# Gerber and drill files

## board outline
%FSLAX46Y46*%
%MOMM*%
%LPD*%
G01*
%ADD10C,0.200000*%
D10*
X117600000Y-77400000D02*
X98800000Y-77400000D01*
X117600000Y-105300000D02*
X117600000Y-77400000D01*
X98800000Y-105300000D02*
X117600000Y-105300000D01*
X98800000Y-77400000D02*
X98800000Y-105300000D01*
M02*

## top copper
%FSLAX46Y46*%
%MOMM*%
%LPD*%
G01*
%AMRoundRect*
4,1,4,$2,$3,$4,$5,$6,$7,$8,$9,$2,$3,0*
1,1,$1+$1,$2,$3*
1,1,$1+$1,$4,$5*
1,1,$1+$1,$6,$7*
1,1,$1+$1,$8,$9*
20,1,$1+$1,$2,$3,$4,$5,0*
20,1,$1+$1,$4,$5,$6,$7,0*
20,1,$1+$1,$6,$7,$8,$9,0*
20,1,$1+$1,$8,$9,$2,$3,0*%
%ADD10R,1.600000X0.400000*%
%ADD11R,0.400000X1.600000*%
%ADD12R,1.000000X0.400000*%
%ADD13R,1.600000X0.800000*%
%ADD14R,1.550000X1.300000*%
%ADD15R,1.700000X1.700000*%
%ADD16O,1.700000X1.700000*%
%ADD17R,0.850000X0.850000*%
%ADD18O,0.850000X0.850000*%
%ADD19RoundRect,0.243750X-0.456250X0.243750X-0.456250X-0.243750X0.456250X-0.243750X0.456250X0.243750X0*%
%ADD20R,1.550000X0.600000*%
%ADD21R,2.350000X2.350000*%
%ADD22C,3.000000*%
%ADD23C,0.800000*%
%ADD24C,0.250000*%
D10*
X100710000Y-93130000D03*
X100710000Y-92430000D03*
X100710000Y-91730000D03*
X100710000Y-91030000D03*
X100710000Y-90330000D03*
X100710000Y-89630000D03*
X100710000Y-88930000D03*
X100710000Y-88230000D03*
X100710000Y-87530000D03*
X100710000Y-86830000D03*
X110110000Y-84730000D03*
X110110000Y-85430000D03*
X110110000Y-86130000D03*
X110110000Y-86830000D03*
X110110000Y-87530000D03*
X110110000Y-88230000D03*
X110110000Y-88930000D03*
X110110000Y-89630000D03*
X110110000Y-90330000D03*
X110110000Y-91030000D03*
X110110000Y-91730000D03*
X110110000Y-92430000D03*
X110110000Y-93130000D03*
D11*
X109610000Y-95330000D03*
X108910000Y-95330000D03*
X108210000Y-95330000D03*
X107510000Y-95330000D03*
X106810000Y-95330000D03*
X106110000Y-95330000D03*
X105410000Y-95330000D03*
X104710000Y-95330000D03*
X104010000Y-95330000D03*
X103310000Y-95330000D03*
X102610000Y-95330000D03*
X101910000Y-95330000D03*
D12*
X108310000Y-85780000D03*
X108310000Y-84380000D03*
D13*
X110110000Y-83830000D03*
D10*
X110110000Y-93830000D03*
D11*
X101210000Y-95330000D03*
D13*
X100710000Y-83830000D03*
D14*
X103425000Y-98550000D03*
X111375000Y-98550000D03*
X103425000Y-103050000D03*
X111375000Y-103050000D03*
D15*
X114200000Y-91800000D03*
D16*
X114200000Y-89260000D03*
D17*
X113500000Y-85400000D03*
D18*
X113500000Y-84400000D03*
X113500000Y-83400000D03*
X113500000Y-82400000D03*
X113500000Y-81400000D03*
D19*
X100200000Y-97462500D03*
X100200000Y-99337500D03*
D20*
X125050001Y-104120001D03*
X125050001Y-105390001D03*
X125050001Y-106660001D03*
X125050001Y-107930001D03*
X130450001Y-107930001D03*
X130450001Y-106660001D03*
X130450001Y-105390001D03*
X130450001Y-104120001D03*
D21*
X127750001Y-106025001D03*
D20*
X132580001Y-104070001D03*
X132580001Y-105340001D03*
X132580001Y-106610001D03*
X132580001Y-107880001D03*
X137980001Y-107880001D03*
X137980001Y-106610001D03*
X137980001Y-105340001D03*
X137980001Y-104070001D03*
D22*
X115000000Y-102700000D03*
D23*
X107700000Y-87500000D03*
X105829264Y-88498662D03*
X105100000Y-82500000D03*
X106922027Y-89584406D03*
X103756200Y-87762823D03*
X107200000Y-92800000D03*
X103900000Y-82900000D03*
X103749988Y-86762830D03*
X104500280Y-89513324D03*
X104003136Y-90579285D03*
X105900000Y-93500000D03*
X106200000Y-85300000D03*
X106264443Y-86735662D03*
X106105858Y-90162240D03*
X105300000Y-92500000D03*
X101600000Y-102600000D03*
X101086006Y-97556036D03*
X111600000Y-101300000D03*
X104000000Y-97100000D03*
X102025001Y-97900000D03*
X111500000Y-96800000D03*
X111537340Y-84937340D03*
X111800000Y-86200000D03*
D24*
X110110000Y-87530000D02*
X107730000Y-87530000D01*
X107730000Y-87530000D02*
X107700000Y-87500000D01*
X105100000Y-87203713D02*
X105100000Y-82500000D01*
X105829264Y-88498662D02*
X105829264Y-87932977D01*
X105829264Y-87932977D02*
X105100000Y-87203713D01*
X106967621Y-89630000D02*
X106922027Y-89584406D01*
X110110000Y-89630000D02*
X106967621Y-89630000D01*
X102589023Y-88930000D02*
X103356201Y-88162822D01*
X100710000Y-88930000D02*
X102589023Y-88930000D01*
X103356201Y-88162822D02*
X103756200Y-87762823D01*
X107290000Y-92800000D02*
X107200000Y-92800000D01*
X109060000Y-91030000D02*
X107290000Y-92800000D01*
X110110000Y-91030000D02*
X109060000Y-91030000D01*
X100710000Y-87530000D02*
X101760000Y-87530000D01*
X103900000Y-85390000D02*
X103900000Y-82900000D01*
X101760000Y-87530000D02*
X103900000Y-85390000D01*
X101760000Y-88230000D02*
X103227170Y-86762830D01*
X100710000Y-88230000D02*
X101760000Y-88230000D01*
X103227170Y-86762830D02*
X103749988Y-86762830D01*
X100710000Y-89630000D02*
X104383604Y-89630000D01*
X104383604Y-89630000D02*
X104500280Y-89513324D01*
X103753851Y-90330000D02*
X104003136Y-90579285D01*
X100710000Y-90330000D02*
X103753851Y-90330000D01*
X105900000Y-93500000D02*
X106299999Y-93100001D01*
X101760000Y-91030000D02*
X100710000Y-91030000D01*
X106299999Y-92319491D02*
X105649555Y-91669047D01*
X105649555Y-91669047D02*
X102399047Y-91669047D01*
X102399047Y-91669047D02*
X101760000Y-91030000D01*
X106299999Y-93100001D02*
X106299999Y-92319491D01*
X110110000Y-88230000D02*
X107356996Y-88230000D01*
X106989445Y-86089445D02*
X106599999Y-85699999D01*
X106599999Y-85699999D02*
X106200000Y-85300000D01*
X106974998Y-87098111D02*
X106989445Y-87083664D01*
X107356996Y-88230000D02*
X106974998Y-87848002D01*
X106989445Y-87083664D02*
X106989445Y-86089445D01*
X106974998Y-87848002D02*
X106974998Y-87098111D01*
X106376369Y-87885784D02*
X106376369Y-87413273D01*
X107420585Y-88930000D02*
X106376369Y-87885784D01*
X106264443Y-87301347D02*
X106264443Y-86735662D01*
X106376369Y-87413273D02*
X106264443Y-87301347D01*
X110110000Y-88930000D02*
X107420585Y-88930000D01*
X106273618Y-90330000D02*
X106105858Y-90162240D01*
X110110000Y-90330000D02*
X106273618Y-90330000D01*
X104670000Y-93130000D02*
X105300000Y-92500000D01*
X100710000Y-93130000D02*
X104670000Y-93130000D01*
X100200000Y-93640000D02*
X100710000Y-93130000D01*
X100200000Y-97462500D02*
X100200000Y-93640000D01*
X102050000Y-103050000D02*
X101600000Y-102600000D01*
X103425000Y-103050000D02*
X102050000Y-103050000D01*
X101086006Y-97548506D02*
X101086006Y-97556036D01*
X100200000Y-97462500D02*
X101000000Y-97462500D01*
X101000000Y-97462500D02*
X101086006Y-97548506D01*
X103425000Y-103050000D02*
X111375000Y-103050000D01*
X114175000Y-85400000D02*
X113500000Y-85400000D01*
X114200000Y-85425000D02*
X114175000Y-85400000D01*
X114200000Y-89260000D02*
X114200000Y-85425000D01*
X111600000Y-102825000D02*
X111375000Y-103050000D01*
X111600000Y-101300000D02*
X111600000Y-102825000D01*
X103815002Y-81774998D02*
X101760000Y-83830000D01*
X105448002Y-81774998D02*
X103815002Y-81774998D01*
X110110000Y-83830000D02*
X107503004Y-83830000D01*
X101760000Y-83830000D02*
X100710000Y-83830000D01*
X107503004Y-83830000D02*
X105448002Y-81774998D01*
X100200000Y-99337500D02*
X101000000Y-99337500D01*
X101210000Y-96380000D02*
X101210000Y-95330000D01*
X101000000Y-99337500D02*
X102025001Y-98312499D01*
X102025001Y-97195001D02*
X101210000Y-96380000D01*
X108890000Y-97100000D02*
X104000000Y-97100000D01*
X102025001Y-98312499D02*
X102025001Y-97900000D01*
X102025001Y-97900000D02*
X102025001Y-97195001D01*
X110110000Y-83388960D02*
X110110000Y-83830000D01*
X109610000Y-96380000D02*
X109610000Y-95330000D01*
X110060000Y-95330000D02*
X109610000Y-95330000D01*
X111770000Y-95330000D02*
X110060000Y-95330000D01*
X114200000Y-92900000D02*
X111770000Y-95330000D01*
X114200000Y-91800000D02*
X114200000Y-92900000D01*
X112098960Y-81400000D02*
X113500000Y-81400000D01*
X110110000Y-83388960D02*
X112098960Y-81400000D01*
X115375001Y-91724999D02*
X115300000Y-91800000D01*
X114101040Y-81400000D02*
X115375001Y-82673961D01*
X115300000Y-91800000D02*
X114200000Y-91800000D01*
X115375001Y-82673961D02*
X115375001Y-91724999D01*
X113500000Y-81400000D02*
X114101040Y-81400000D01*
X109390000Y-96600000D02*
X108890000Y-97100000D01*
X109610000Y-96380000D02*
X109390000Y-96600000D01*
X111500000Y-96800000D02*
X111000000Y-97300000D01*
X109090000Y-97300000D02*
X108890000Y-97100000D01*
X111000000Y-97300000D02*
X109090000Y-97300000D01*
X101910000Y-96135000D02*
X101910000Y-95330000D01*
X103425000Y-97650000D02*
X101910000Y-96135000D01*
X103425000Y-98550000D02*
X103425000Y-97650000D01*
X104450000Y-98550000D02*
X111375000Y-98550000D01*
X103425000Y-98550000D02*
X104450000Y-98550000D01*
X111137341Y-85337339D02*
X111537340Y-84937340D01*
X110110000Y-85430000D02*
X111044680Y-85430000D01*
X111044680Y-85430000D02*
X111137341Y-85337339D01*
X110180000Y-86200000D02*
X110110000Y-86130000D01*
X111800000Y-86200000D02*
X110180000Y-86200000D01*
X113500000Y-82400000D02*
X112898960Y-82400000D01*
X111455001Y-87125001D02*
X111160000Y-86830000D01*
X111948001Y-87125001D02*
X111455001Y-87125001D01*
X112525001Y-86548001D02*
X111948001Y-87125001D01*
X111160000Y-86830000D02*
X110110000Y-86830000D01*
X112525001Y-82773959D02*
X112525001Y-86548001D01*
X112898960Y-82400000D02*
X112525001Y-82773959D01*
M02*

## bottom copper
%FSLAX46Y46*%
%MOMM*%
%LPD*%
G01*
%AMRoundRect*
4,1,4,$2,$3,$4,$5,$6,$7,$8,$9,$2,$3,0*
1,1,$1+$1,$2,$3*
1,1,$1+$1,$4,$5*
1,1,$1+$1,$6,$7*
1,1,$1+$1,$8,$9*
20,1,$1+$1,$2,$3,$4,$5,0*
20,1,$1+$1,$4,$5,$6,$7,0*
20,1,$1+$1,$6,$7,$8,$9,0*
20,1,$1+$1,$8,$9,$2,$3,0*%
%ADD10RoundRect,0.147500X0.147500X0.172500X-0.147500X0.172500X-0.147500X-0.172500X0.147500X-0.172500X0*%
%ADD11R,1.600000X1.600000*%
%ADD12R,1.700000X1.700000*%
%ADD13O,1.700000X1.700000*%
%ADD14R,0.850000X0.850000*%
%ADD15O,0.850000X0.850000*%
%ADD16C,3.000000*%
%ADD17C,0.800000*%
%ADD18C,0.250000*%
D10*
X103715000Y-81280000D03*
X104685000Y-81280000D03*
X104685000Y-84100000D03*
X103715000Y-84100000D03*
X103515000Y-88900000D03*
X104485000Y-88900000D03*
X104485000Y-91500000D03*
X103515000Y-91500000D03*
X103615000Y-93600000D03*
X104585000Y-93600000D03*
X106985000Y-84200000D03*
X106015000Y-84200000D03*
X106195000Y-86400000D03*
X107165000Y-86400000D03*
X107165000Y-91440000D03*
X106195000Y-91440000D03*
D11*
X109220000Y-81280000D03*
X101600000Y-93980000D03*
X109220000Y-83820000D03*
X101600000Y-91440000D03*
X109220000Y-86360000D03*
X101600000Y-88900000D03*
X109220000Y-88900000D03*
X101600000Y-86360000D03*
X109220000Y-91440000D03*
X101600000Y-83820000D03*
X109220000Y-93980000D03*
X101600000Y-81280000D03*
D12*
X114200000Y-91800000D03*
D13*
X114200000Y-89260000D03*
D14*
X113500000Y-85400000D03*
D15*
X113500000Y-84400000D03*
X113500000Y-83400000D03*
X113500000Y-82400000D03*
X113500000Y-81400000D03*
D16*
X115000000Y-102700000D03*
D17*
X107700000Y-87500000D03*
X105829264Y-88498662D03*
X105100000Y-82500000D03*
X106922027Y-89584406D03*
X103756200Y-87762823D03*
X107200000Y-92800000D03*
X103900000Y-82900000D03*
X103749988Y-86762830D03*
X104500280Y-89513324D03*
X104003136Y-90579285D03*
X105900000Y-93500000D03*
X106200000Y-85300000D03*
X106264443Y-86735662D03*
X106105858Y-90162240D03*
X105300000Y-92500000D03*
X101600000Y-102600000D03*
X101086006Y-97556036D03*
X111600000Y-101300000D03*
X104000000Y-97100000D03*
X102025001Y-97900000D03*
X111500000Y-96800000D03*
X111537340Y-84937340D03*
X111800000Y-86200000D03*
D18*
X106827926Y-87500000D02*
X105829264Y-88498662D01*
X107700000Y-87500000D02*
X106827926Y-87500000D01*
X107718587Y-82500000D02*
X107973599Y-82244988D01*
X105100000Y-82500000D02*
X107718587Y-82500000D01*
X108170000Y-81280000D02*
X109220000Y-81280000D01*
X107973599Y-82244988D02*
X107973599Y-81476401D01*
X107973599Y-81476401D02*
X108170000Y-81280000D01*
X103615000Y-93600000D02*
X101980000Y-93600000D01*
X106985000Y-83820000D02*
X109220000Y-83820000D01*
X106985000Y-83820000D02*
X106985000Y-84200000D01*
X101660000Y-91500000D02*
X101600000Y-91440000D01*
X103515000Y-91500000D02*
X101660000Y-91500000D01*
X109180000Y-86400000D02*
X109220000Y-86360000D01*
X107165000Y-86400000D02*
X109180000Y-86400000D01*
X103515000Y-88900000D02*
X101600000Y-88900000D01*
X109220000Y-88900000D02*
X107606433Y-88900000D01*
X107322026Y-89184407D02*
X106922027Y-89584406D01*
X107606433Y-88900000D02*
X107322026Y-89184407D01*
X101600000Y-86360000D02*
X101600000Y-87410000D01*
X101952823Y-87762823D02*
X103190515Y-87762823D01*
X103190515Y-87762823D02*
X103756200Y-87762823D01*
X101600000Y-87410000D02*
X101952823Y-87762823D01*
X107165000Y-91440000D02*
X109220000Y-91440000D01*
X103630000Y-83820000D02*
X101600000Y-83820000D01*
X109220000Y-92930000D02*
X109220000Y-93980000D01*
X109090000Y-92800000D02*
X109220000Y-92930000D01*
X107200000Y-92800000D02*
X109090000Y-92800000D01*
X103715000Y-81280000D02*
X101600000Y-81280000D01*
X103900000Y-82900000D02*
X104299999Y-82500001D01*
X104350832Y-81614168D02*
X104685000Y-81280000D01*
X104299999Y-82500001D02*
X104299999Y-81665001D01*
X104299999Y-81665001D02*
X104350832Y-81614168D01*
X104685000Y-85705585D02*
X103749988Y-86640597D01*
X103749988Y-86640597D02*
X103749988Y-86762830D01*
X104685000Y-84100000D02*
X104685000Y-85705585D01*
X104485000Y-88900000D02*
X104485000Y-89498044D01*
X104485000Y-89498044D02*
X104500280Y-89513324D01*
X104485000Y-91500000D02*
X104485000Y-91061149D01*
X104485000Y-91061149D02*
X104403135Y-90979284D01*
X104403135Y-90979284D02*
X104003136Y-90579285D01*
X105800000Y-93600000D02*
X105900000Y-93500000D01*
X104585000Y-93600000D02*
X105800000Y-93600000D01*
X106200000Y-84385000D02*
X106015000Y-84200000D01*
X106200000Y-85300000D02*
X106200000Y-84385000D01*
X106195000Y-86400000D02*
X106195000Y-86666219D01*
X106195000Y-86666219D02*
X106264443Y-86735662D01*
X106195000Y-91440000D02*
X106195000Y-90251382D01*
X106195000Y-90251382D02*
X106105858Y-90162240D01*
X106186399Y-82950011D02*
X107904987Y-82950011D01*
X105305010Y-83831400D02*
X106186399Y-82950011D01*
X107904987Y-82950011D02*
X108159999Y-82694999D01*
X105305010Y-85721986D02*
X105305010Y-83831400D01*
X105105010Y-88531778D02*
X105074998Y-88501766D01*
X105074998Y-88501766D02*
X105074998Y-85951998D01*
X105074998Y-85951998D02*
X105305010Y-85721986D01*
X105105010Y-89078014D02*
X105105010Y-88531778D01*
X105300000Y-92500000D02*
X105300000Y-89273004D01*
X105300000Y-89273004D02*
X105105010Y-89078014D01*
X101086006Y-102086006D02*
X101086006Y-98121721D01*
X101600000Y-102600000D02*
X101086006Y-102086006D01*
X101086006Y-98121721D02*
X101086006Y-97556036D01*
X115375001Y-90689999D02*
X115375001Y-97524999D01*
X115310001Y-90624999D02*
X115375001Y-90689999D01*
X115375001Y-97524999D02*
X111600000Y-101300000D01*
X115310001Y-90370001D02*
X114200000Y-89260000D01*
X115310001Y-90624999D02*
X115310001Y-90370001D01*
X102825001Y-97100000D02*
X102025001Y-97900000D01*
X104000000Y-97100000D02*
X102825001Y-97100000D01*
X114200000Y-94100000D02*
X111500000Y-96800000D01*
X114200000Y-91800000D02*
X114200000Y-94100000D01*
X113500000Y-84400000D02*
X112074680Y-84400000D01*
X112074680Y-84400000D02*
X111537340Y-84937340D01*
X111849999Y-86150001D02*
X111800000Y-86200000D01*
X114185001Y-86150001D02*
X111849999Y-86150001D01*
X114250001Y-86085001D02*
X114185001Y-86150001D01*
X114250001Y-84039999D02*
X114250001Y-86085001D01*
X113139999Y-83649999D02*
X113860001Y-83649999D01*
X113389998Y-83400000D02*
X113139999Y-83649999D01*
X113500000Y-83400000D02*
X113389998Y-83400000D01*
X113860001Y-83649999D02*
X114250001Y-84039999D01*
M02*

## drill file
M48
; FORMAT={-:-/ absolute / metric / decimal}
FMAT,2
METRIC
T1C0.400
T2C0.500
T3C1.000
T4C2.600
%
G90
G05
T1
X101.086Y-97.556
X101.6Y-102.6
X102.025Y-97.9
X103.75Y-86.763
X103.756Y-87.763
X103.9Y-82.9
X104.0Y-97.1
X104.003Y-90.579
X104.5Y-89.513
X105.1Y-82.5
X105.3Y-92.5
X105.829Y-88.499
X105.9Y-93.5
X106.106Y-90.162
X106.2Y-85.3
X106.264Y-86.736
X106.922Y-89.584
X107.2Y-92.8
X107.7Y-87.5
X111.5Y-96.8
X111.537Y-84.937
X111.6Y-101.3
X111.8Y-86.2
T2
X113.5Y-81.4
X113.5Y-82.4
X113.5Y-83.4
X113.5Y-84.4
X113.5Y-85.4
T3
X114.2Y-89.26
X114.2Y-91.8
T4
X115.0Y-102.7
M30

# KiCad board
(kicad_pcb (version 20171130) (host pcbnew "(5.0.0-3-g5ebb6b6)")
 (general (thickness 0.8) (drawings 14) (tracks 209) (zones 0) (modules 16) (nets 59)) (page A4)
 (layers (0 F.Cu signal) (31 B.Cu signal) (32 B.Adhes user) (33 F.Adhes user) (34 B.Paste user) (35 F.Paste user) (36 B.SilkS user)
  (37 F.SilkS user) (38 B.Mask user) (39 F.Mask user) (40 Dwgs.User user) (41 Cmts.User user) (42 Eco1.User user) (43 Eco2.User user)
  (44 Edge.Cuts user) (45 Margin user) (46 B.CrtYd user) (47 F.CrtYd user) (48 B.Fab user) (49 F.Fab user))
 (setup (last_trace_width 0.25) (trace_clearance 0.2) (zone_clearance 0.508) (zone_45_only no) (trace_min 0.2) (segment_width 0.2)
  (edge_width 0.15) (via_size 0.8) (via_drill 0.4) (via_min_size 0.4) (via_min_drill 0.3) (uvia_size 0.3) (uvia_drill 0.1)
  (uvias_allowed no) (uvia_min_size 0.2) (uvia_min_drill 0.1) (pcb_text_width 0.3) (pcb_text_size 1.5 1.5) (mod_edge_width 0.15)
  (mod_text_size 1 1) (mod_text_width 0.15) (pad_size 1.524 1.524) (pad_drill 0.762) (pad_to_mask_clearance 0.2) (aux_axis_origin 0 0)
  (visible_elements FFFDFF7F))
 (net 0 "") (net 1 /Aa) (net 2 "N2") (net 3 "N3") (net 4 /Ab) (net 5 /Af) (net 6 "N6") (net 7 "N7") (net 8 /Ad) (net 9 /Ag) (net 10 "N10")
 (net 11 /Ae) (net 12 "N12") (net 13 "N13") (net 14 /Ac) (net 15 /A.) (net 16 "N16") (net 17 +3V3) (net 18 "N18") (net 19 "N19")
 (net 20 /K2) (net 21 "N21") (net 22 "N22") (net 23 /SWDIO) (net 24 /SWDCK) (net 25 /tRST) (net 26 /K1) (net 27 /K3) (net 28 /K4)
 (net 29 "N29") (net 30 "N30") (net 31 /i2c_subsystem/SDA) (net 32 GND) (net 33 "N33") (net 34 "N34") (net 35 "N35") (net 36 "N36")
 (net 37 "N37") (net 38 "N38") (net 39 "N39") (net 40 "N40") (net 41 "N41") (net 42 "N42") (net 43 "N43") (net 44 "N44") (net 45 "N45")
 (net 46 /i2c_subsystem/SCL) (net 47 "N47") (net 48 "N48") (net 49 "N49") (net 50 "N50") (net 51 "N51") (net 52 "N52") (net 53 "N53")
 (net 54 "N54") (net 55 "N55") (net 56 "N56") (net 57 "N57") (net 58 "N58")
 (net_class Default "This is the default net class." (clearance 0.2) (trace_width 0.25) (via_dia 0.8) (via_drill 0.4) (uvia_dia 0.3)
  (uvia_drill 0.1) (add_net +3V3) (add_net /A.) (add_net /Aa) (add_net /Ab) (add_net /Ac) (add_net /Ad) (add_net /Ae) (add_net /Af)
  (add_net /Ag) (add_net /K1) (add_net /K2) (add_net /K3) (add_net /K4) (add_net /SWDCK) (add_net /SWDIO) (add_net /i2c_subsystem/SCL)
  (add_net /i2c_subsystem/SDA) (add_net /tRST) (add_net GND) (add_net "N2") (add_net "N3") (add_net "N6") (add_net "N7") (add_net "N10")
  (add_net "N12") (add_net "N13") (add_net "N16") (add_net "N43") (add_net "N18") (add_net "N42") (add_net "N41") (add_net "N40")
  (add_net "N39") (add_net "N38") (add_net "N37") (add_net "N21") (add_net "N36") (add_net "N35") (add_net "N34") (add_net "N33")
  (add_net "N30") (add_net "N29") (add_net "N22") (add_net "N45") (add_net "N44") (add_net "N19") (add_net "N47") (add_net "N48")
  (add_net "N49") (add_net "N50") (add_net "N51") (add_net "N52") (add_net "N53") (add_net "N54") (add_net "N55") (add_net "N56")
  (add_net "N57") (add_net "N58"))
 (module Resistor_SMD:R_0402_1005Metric (layer B.Cu) (at 104.2 81.28 180)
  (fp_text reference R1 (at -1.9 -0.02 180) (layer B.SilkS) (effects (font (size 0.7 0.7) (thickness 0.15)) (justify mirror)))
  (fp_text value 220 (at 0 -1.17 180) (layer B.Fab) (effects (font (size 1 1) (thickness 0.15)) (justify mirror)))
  (pad 2 smd roundrect (at 0.485 0 180) (size 0.59 0.64) (layers B.Cu B.Paste B.Mask) (roundrect_rratio 0.25) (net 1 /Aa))
  (pad 1 smd roundrect (at -0.485 0 180) (size 0.59 0.64) (layers B.Cu B.Paste B.Mask) (roundrect_rratio 0.25) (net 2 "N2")))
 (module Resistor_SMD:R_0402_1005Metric (layer B.Cu) (at 104.2 84.1 180)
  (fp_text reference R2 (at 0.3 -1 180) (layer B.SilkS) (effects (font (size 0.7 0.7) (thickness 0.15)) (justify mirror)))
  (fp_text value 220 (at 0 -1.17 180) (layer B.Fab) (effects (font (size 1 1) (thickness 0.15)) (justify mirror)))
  (pad 1 smd roundrect (at -0.485 0 180) (size 0.59 0.64) (layers B.Cu B.Paste B.Mask) (roundrect_rratio 0.25) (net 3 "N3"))
  (pad 2 smd roundrect (at 0.485 0 180) (size 0.59 0.64) (layers B.Cu B.Paste B.Mask) (roundrect_rratio 0.25) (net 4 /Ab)))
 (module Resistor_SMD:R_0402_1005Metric (layer B.Cu) (at 104 88.9 180)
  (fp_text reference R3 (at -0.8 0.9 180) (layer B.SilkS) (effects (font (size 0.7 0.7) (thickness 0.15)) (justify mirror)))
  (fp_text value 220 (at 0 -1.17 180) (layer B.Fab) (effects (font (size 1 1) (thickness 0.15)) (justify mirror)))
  (pad 2 smd roundrect (at 0.485 0 180) (size 0.59 0.64) (layers B.Cu B.Paste B.Mask) (roundrect_rratio 0.25) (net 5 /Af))
  (pad 1 smd roundrect (at -0.485 0 180) (size 0.59 0.64) (layers B.Cu B.Paste B.Mask) (roundrect_rratio 0.25) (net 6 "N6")))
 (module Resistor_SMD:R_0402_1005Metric (layer B.Cu) (at 104 91.5 180)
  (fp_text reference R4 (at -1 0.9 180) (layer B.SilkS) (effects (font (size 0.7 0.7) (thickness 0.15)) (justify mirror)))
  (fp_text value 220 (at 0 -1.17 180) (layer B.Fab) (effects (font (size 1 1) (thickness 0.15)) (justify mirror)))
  (pad 1 smd roundrect (at -0.485 0 180) (size 0.59 0.64) (layers B.Cu B.Paste B.Mask) (roundrect_rratio 0.25) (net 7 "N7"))
  (pad 2 smd roundrect (at 0.485 0 180) (size 0.59 0.64) (layers B.Cu B.Paste B.Mask) (roundrect_rratio 0.25) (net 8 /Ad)))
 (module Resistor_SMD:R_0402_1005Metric (layer B.Cu) (at 104.1 93.6 180)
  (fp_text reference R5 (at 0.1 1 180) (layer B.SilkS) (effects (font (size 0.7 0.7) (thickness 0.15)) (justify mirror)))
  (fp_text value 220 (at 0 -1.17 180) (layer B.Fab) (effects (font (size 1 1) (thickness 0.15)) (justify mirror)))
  (pad 2 smd roundrect (at 0.485 0 180) (size 0.59 0.64) (layers B.Cu B.Paste B.Mask) (roundrect_rratio 0.25) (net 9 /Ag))
  (pad 1 smd roundrect (at -0.485 0 180) (size 0.59 0.64) (layers B.Cu B.Paste B.Mask) (roundrect_rratio 0.25) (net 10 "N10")))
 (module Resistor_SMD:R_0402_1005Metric (layer B.Cu) (at 106.5 84.2 180)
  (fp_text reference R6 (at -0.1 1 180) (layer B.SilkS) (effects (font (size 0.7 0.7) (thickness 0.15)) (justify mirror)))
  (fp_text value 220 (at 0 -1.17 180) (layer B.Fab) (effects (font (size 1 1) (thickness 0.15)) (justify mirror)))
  (pad 1 smd roundrect (at -0.485 0 180) (size 0.59 0.64) (layers B.Cu B.Paste B.Mask) (roundrect_rratio 0.25) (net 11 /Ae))
  (pad 2 smd roundrect (at 0.485 0 180) (size 0.59 0.64) (layers B.Cu B.Paste B.Mask) (roundrect_rratio 0.25) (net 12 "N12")))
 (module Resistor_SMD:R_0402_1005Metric (layer B.Cu) (at 106.68 86.4 180)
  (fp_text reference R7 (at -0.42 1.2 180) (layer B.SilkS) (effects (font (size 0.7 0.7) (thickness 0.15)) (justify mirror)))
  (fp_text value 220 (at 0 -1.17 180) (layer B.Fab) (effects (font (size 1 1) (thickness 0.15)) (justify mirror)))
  (pad 2 smd roundrect (at 0.485 0 180) (size 0.59 0.64) (layers B.Cu B.Paste B.Mask) (roundrect_rratio 0.25) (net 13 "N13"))
  (pad 1 smd roundrect (at -0.485 0 180) (size 0.59 0.64) (layers B.Cu B.Paste B.Mask) (roundrect_rratio 0.25) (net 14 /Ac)))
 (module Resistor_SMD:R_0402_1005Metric (layer B.Cu) (at 106.68 91.44 180)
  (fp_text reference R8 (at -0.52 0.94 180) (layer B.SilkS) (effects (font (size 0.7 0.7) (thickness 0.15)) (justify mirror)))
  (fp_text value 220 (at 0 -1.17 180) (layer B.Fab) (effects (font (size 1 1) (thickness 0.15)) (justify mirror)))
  (pad 1 smd roundrect (at -0.485 0 180) (size 0.59 0.64) (layers B.Cu B.Paste B.Mask) (roundrect_rratio 0.25) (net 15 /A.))
  (pad 2 smd roundrect (at 0.485 0 180) (size 0.59 0.64) (layers B.Cu B.Paste B.Mask) (roundrect_rratio 0.25) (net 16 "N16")))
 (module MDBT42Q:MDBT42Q (layer F.Cu) (at 105.41 87.63)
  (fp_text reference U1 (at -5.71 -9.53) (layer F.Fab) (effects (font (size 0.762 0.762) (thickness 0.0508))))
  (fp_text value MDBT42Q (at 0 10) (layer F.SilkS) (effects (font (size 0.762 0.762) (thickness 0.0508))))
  (pad 11 smd rect (at -4.7 5.5) (size 1.6 0.4) (layers F.Cu F.Paste F.Mask) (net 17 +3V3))
  (pad 10 smd rect (at -4.7 4.8) (size 1.6 0.4) (layers F.Cu F.Paste F.Mask) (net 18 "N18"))
  (pad 9 smd rect (at -4.7 4.1) (size 1.6 0.4) (layers F.Cu F.Paste F.Mask) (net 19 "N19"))
  (pad 8 smd rect (at -4.7 3.4) (size 1.6 0.4) (layers F.Cu F.Paste F.Mask) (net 10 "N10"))
  (pad 7 smd rect (at -4.7 2.7) (size 1.6 0.4) (layers F.Cu F.Paste F.Mask) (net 7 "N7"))
  (pad 6 smd rect (at -4.7 2) (size 1.6 0.4) (layers F.Cu F.Paste F.Mask) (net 6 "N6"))
  (pad 5 smd rect (at -4.7 1.3) (size 1.6 0.4) (layers F.Cu F.Paste F.Mask) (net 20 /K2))
  (pad 4 smd rect (at -4.7 0.6) (size 1.6 0.4) (layers F.Cu F.Paste F.Mask) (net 3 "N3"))
  (pad 3 smd rect (at -4.7 -0.1) (size 1.6 0.4) (layers F.Cu F.Paste F.Mask) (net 2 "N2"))
  (pad 2 smd rect (at -4.7 -0.8) (size 1.6 0.4) (layers F.Cu F.Paste F.Mask) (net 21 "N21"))
  (pad 38 smd rect (at 4.7 -2.9 180) (size 1.6 0.4) (layers F.Cu F.Paste F.Mask) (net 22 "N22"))
  (pad 37 smd rect (at 4.7 -2.2 180) (size 1.6 0.4) (layers F.Cu F.Paste F.Mask) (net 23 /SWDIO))
  (pad 36 smd rect (at 4.7 -1.5 180) (size 1.6 0.4) (layers F.Cu F.Paste F.Mask) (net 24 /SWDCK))
  (pad 35 smd rect (at 4.7 -0.8 180) (size 1.6 0.4) (layers F.Cu F.Paste F.Mask) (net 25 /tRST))
  (pad 34 smd rect (at 4.7 -0.1 180) (size 1.6 0.4) (layers F.Cu F.Paste F.Mask) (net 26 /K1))
  (pad 33 smd rect (at 4.7 0.6 180) (size 1.6 0.4) (layers F.Cu F.Paste F.Mask) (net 12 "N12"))
  (pad 32 smd rect (at 4.7 1.3 180) (size 1.6 0.4) (layers F.Cu F.Paste F.Mask) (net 13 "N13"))
  (pad 31 smd rect (at 4.7 2 180) (size 1.6 0.4) (layers F.Cu F.Paste F.Mask) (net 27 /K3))
  (pad 30 smd rect (at 4.7 2.7 180) (size 1.6 0.4) (layers F.Cu F.Paste F.Mask) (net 16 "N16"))
  (pad 29 smd rect (at 4.7 3.4 180) (size 1.6 0.4) (layers F.Cu F.Paste F.Mask) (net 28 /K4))
  (pad 28 smd rect (at 4.7 4.1 180) (size 1.6 0.4) (layers F.Cu F.Paste F.Mask) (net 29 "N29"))
  (pad 27 smd rect (at 4.7 4.8 180) (size 1.6 0.4) (layers F.Cu F.Paste F.Mask) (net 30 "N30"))
  (pad 26 smd rect (at 4.7 5.5 180) (size 1.6 0.4) (layers F.Cu F.Paste F.Mask) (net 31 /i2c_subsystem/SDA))
  (pad 24 smd rect (at 4.2 7.7 90) (size 1.6 0.4) (layers F.Cu F.Paste F.Mask) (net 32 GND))
  (pad 23 smd rect (at 3.5 7.7 90) (size 1.6 0.4) (layers F.Cu F.Paste F.Mask) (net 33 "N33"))
  (pad 22 smd rect (at 2.8 7.7 90) (size 1.6 0.4) (layers F.Cu F.Paste F.Mask) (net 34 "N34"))
  (pad 21 smd rect (at 2.1 7.7 90) (size 1.6 0.4) (layers F.Cu F.Paste F.Mask) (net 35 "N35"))
  (pad 20 smd rect (at 1.4 7.7 90) (size 1.6 0.4) (layers F.Cu F.Paste F.Mask) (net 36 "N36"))
  (pad 19 smd rect (at 0.7 7.7 90) (size 1.6 0.4) (layers F.Cu F.Paste F.Mask) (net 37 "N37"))
  (pad 18 smd rect (at 0 7.7 90) (size 1.6 0.4) (layers F.Cu F.Paste F.Mask) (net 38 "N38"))
  (pad 17 smd rect (at -0.7 7.7 90) (size 1.6 0.4) (layers F.Cu F.Paste F.Mask) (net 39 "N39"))
  (pad 16 smd rect (at -1.4 7.7 90) (size 1.6 0.4) (layers F.Cu F.Paste F.Mask) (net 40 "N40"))
  (pad 15 smd rect (at -2.1 7.7 90) (size 1.6 0.4) (layers F.Cu F.Paste F.Mask) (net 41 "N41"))
  (pad 14 smd rect (at -2.8 7.7 90) (size 1.6 0.4) (layers F.Cu F.Paste F.Mask) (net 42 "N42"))
  (pad 13 smd rect (at -3.5 7.7 90) (size 1.6 0.4) (layers F.Cu F.Paste F.Mask) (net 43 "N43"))
  (pad 41 smd rect (at 2.9 -1.85 180) (size 1 0.4) (layers F.Cu F.Paste F.Mask) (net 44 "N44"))
  (pad 40 smd rect (at 2.9 -3.25 180) (size 1 0.4) (layers F.Cu F.Paste F.Mask) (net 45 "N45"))
  (pad 39 smd rect (at 4.7 -3.8 180) (size 1.6 0.8) (layers F.Cu F.Paste F.Mask) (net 32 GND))
  (pad 25 smd rect (at 4.7 6.2 180) (size 1.6 0.4) (layers F.Cu F.Paste F.Mask) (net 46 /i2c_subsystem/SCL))
  (pad 12 smd rect (at -4.2 7.7 90) (size 1.6 0.4) (layers F.Cu F.Paste F.Mask) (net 32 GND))
  (pad 1 smd rect (at -4.7 -3.8) (size 1.6 0.8) (layers F.Cu F.Paste F.Mask) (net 32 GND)))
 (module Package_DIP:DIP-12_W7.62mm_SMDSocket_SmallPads (layer B.Cu) (at 105.41 87.63 180)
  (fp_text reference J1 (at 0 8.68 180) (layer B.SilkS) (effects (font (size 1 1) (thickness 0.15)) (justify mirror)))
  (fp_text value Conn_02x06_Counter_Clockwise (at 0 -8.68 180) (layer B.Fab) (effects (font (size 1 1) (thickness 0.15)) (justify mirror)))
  (pad 1 smd rect (at -3.81 6.35 180) (size 1.6 1.6) (layers B.Cu B.Paste B.Mask) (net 26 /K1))
  (pad 7 smd rect (at 3.81 -6.35 180) (size 1.6 1.6) (layers B.Cu B.Paste B.Mask) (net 9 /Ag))
  (pad 2 smd rect (at -3.81 3.81 180) (size 1.6 1.6) (layers B.Cu B.Paste B.Mask) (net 11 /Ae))
  (pad 8 smd rect (at 3.81 -3.81 180) (size 1.6 1.6) (layers B.Cu B.Paste B.Mask) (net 8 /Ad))
  (pad 3 smd rect (at -3.81 1.27 180) (size 1.6 1.6) (layers B.Cu B.Paste B.Mask) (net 14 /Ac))
  (pad 9 smd rect (at 3.81 -1.27 180) (size 1.6 1.6) (layers B.Cu B.Paste B.Mask) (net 5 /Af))
  (pad 4 smd rect (at -3.81 -1.27 180) (size 1.6 1.6) (layers B.Cu B.Paste B.Mask) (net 27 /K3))
  (pad 10 smd rect (at 3.81 1.27 180) (size 1.6 1.6) (layers B.Cu B.Paste B.Mask) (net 20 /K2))
  (pad 5 smd rect (at -3.81 -3.81 180) (size 1.6 1.6) (layers B.Cu B.Paste B.Mask) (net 15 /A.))
  (pad 11 smd rect (at 3.81 3.81 180) (size 1.6 1.6) (layers B.Cu B.Paste B.Mask) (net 4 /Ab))
  (pad 6 smd rect (at -3.81 -6.35 180) (size 1.6 1.6) (layers B.Cu B.Paste B.Mask) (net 28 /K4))
  (pad 12 smd rect (at 3.81 6.35 180) (size 1.6 1.6) (layers B.Cu B.Paste B.Mask) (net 1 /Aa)))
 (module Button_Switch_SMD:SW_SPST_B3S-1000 (layer F.Cu) (at 107.4 100.8)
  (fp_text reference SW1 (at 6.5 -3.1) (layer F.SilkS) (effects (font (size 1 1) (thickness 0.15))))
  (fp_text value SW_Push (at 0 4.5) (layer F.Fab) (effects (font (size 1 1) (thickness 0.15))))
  (pad 1 smd rect (at -3.975 -2.25) (size 1.55 1.3) (layers F.Cu F.Paste F.Mask) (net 43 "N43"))
  (pad 1 smd rect (at 3.975 -2.25) (size 1.55 1.3) (layers F.Cu F.Paste F.Mask) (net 43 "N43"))
  (pad 2 smd rect (at -3.975 2.25) (size 1.55 1.3) (layers F.Cu F.Paste F.Mask) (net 17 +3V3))
  (pad 2 smd rect (at 3.975 2.25) (size 1.55 1.3) (layers F.Cu F.Paste F.Mask) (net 17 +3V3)))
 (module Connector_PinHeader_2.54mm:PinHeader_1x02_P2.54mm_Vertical (layer F.Cu) (at 114.2 91.8 180)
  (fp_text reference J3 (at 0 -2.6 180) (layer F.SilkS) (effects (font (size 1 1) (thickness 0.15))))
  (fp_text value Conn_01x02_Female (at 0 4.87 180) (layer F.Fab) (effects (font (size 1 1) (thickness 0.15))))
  (pad 1 thru_hole rect (at 0 0 180) (size 1.7 1.7) (drill 1) (layers *.Cu *.Mask) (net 32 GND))
  (pad 2 thru_hole oval (at 0 2.54 180) (size 1.7 1.7) (drill 1) (layers *.Cu *.Mask) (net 17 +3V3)))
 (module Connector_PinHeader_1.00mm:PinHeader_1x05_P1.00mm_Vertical (layer F.Cu) (at 113.5 85.4 180)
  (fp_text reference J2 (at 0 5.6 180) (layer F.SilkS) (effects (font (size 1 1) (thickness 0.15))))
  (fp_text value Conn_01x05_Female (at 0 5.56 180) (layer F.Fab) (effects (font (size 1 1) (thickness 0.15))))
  (pad 1 thru_hole rect (at 0 0 180) (size 0.85 0.85) (drill 0.5) (layers *.Cu *.Mask) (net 17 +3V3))
  (pad 2 thru_hole oval (at 0 1 180) (size 0.85 0.85) (drill 0.5) (layers *.Cu *.Mask) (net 23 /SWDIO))
  (pad 3 thru_hole oval (at 0 2 180) (size 0.85 0.85) (drill 0.5) (layers *.Cu *.Mask) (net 24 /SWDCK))
  (pad 4 thru_hole oval (at 0 3 180) (size 0.85 0.85) (drill 0.5) (layers *.Cu *.Mask) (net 25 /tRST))
  (pad 5 thru_hole oval (at 0 4 180) (size 0.85 0.85) (drill 0.5) (layers *.Cu *.Mask) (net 32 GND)))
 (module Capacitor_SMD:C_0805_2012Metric (layer F.Cu) (at 100.2 98.4 270)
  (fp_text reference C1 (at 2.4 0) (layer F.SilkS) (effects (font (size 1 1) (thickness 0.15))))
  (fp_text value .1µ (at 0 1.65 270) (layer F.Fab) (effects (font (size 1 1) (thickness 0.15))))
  (pad 1 smd roundrect (at -0.9375 0 270) (size 0.975 1.4) (layers F.Cu F.Paste F.Mask) (roundrect_rratio 0.25) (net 17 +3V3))
  (pad 2 smd roundrect (at 0.9375 0 270) (size 0.975 1.4) (layers F.Cu F.Paste F.Mask) (roundrect_rratio 0.25) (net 32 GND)))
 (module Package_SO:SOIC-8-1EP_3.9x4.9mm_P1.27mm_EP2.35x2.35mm (layer F.Cu) (at 127.750001 106.025001)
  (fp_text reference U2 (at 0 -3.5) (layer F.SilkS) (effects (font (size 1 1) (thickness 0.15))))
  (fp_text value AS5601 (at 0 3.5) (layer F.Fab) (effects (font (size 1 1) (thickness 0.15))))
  (pad 1 smd rect (at -2.7 -1.905) (size 1.55 0.6) (layers F.Cu F.Paste F.Mask) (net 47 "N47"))
  (pad 2 smd rect (at -2.7 -0.635) (size 1.55 0.6) (layers F.Cu F.Paste F.Mask) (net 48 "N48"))
  (pad 3 smd rect (at -2.7 0.635) (size 1.55 0.6) (layers F.Cu F.Paste F.Mask) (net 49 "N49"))
  (pad 4 smd rect (at -2.7 1.905) (size 1.55 0.6) (layers F.Cu F.Paste F.Mask) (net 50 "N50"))
  (pad 5 smd rect (at 2.7 1.905) (size 1.55 0.6) (layers F.Cu F.Paste F.Mask) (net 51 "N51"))
  (pad 6 smd rect (at 2.7 0.635) (size 1.55 0.6) (layers F.Cu F.Paste F.Mask) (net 31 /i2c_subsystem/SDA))
  (pad 7 smd rect (at 2.7 -0.635) (size 1.55 0.6) (layers F.Cu F.Paste F.Mask) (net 46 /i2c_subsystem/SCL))
  (pad 8 smd rect (at 2.7 -1.905) (size 1.55 0.6) (layers F.Cu F.Paste F.Mask) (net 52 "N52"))
  (pad "" smd rect (at 0.5875 0.5875) (size 0.95 0.95) (layers F.Paste))
  (pad 9 smd rect (at 0 0) (size 2.35 2.35) (layers F.Cu F.Mask))
  (pad "" smd rect (at -0.5875 0.5875) (size 0.95 0.95) (layers F.Paste))
  (pad "" smd rect (at -0.5875 -0.5875) (size 0.95 0.95) (layers F.Paste))
  (pad "" smd rect (at 0.5875 -0.5875) (size 0.95 0.95) (layers F.Paste)))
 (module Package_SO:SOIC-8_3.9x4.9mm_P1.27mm (layer F.Cu) (at 135.280001 105.975001)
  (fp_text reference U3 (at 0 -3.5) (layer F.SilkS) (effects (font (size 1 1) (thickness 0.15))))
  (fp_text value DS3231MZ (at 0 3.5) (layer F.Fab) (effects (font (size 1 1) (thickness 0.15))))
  (pad 1 smd rect (at -2.7 -1.905) (size 1.55 0.6) (layers F.Cu F.Paste F.Mask) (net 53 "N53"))
  (pad 2 smd rect (at -2.7 -0.635) (size 1.55 0.6) (layers F.Cu F.Paste F.Mask) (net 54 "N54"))
  (pad 3 smd rect (at -2.7 0.635) (size 1.55 0.6) (layers F.Cu F.Paste F.Mask) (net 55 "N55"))
  (pad 4 smd rect (at -2.7 1.905) (size 1.55 0.6) (layers F.Cu F.Paste F.Mask) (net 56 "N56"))
  (pad 5 smd rect (at 2.7 1.905) (size 1.55 0.6) (layers F.Cu F.Paste F.Mask) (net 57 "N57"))
  (pad 6 smd rect (at 2.7 0.635) (size 1.55 0.6) (layers F.Cu F.Paste F.Mask) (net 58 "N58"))
  (pad 7 smd rect (at 2.7 -0.635) (size 1.55 0.6) (layers F.Cu F.Paste F.Mask) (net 31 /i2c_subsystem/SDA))
  (pad 8 smd rect (at 2.7 -1.905) (size 1.55 0.6) (layers F.Cu F.Paste F.Mask) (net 46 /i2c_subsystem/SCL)))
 (gr_line (start 117.6 77.4) (end 98.8 77.4) (layer Edge.Cuts) (width 0.2))
 (gr_line (start 117.6 105.3) (end 117.6 77.4) (layer Edge.Cuts) (width 0.2))
 (gr_line (start 98.8 105.3) (end 117.6 105.3) (layer Edge.Cuts) (width 0.2))
 (gr_line (start 98.8 77.4) (end 98.8 105.3) (layer Edge.Cuts) (width 0.2))
 (via (at 115 102.7) (size 3) (drill 2.6) (layers F.Cu B.Cu) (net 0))
 (via (at 107.7 87.5) (size 0.8) (drill 0.4) (layers F.Cu B.Cu) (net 26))
 (segment (start 110.11 87.53) (end 107.73 87.53) (width 0.25) (layer F.Cu) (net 26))
 (segment (start 107.73 87.53) (end 107.7 87.5) (width 0.25) (layer F.Cu) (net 26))
 (segment (start 106.827926 87.5) (end 105.829264 88.498662) (width 0.25) (layer B.Cu) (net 26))
 (via (at 105.829264 88.498662) (size 0.8) (drill 0.4) (layers F.Cu B.Cu) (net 26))
 (segment (start 107.7 87.5) (end 106.827926 87.5) (width 0.25) (layer B.Cu) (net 26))
 (via (at 105.1 82.5) (size 0.8) (drill 0.4) (layers F.Cu B.Cu) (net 26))
 (segment (start 105.1 87.203713) (end 105.1 82.5) (width 0.25) (layer F.Cu) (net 26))
 (segment (start 105.829264 88.498662) (end 105.829264 87.932977) (width 0.25) (layer F.Cu) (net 26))
 (segment (start 105.829264 87.932977) (end 105.1 87.203713) (width 0.25) (layer F.Cu) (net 26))
 (segment (start 107.718587 82.5) (end 107.973599 82.244988) (width 0.25) (layer B.Cu) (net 26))
 (segment (start 105.1 82.5) (end 107.718587 82.5) (width 0.25) (layer B.Cu) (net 26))
 (segment (start 108.17 81.28) (end 109.22 81.28) (width 0.25) (layer B.Cu) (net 26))
 (segment (start 107.973599 82.244988) (end 107.973599 81.476401) (width 0.25) (layer B.Cu) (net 26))
 (segment (start 107.973599 81.476401) (end 108.17 81.28) (width 0.25) (layer B.Cu) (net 26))
 (segment (start 103.615 93.6) (end 101.98 93.6) (width 0.25) (layer B.Cu) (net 9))
 (segment (start 106.985 83.82) (end 109.22 83.82) (width 0.25) (layer B.Cu) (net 11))
 (segment (start 106.985 83.82) (end 106.985 84.2) (width 0.25) (layer B.Cu) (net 11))
 (segment (start 101.66 91.5) (end 101.6 91.44) (width 0.25) (layer B.Cu) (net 8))
 (segment (start 103.515 91.5) (end 101.66 91.5) (width 0.25) (layer B.Cu) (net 8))
 (segment (start 109.18 86.4) (end 109.22 86.36) (width 0.25) (layer B.Cu) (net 14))
 (segment (start 107.165 86.4) (end 109.18 86.4) (width 0.25) (layer B.Cu) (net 14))
 (segment (start 103.515 88.9) (end 101.6 88.9) (width 0.25) (layer B.Cu) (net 5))
 (segment (start 106.967621 89.63) (end 106.922027 89.584406) (width 0.25) (layer F.Cu) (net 27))
 (segment (start 109.22 88.9) (end 107.606433 88.9) (width 0.25) (layer B.Cu) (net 27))
 (segment (start 110.11 89.63) (end 106.967621 89.63) (width 0.25) (layer F.Cu) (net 27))
 (segment (start 107.322026 89.184407) (end 106.922027 89.584406) (width 0.25) (layer B.Cu) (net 27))
 (via (at 106.922027 89.584406) (size 0.8) (drill 0.4) (layers F.Cu B.Cu) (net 27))
 (segment (start 107.606433 88.9) (end 107.322026 89.184407) (width 0.25) (layer B.Cu) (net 27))
 (segment (start 101.6 86.36) (end 101.6 87.41) (width 0.25) (layer B.Cu) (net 20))
 (segment (start 102.589023 88.93) (end 103.356201 88.162822) (width 0.25) (layer F.Cu) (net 20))
 (via (at 103.7562 87.762823) (size 0.8) (drill 0.4) (layers F.Cu B.Cu) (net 20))
 (segment (start 101.952823 87.762823) (end 103.190515 87.762823) (width 0.25) (layer B.Cu) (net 20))
 (segment (start 100.71 88.93) (end 102.589023 88.93) (width 0.25) (layer F.Cu) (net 20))
 (segment (start 103.356201 88.162822) (end 103.7562 87.762823) (width 0.25) (layer F.Cu) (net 20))
 (segment (start 103.190515 87.762823) (end 103.7562 87.762823) (width 0.25) (layer B.Cu) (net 20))
 (segment (start 101.6 87.41) (end 101.952823 87.762823) (width 0.25) (layer B.Cu) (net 20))
 (segment (start 107.165 91.44) (end 109.22 91.44) (width 0.25) (layer B.Cu) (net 15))
 (segment (start 103.63 83.82) (end 101.6 83.82) (width 0.25) (layer B.Cu) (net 4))
 (via (at 107.2 92.8) (size 0.8) (drill 0.4) (layers F.Cu B.Cu) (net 28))
 (segment (start 107.29 92.8) (end 107.2 92.8) (width 0.25) (layer F.Cu) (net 28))
 (segment (start 109.06 91.03) (end 107.29 92.8) (width 0.25) (layer F.Cu) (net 28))
 (segment (start 110.11 91.03) (end 109.06 91.03) (width 0.25) (layer F.Cu) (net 28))
 (segment (start 109.22 92.93) (end 109.22 93.98) (width 0.25) (layer B.Cu) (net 28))
 (segment (start 109.09 92.8) (end 109.22 92.93) (width 0.25) (layer B.Cu) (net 28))
 (segment (start 107.2 92.8) (end 109.09 92.8) (width 0.25) (layer B.Cu) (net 28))
 (segment (start 103.715 81.28) (end 101.6 81.28) (width 0.25) (layer B.Cu) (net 1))
 (via (at 103.9 82.9) (size 0.8) (drill 0.4) (layers F.Cu B.Cu) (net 2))
 (segment (start 100.71 87.53) (end 101.76 87.53) (width 0.25) (layer F.Cu) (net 2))
 (segment (start 103.9 85.39) (end 103.9 82.9) (width 0.25) (layer F.Cu) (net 2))
 (segment (start 101.76 87.53) (end 103.9 85.39) (width 0.25) (layer F.Cu) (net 2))
 (segment (start 103.9 82.9) (end 104.299999 82.500001) (width 0.25) (layer B.Cu) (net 2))
 (segment (start 104.350832 81.614168) (end 104.685 81.28) (width 0.25) (layer B.Cu) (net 2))
 (segment (start 104.299999 82.500001) (end 104.299999 81.665001) (width 0.25) (layer B.Cu) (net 2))
 (segment (start 104.299999 81.665001) (end 104.350832 81.614168) (width 0.25) (layer B.Cu) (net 2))
 (via (at 103.749988 86.76283) (size 0.8) (drill 0.4) (layers F.Cu B.Cu) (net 3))
 (segment (start 104.685 85.705585) (end 103.749988 86.640597) (width 0.25) (layer B.Cu) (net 3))
 (segment (start 101.76 88.23) (end 103.22717 86.76283) (width 0.25) (layer F.Cu) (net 3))
 (segment (start 100.71 88.23) (end 101.76 88.23) (width 0.25) (layer F.Cu) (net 3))
 (segment (start 103.749988 86.640597) (end 103.749988 86.76283) (width 0.25) (layer B.Cu) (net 3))
 (segment (start 103.22717 86.76283) (end 103.749988 86.76283) (width 0.25) (layer F.Cu) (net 3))
 (segment (start 104.685 84.1) (end 104.685 85.705585) (width 0.25) (layer B.Cu) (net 3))
 (segment (start 100.71 89.63) (end 104.383604 89.63) (width 0.25) (layer F.Cu) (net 6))
 (segment (start 104.485 88.9) (end 104.485 89.498044) (width 0.25) (layer B.Cu) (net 6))
 (segment (start 104.485 89.498044) (end 104.50028 89.513324) (width 0.25) (layer B.Cu) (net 6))
 (via (at 104.50028 89.513324) (size 0.8) (drill 0.4) (layers F.Cu B.Cu) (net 6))
 (segment (start 104.383604 89.63) (end 104.50028 89.513324) (width 0.25) (layer F.Cu) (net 6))
 (segment (start 103.753851 90.33) (end 104.003136 90.579285) (width 0.25) (layer F.Cu) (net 7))
 (segment (start 104.485 91.5) (end 104.485 91.061149) (width 0.25) (layer B.Cu) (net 7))
 (segment (start 104.485 91.061149) (end 104.403135 90.979284) (width 0.25) (layer B.Cu) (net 7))
 (via (at 104.003136 90.579285) (size 0.8) (drill 0.4) (layers F.Cu B.Cu) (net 7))
 (segment (start 104.403135 90.979284) (end 104.003136 90.579285) (width 0.25) (layer B.Cu) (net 7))
 (segment (start 100.71 90.33) (end 103.753851 90.33) (width 0.25) (layer F.Cu) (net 7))
 (segment (start 105.8 93.6) (end 105.9 93.5) (width 0.25) (layer B.Cu) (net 10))
 (via (at 105.9 93.5) (size 0.8) (drill 0.4) (layers F.Cu B.Cu) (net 10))
 (segment (start 104.585 93.6) (end 105.8 93.6) (width 0.25) (layer B.Cu) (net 10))
 (segment (start 105.9 93.5) (end 106.299999 93.100001) (width 0.25) (layer F.Cu) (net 10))
 (segment (start 101.76 91.03) (end 100.71 91.03) (width 0.25) (layer F.Cu) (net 10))
 (segment (start 106.299999 92.319491) (end 105.649555 91.669047) (width 0.25) (layer F.Cu) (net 10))
 (segment (start 105.649555 91.669047) (end 102.399047 91.669047) (width 0.25) (layer F.Cu) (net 10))
 (segment (start 102.399047 91.669047) (end 101.76 91.03) (width 0.25) (layer F.Cu) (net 10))
 (segment (start 106.299999 93.100001) (end 106.299999 92.319491) (width 0.25) (layer F.Cu) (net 10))
 (via (at 106.2 85.3) (size 0.8) (drill 0.4) (layers F.Cu B.Cu) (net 12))
 (segment (start 106.2 84.385) (end 106.015 84.2) (width 0.25) (layer B.Cu) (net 12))
 (segment (start 106.2 85.3) (end 106.2 84.385) (width 0.25) (layer B.Cu) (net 12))
 (segment (start 110.11 88.23) (end 107.356996 88.23) (width 0.25) (layer F.Cu) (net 12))
 (segment (start 106.989445 86.089445) (end 106.599999 85.699999) (width 0.25) (layer F.Cu) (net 12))
 (segment (start 106.599999 85.699999) (end 106.2 85.3) (width 0.25) (layer F.Cu) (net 12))
 (segment (start 106.974998 87.098111) (end 106.989445 87.083664) (width 0.25) (layer F.Cu) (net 12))
 (segment (start 107.356996 88.23) (end 106.974998 87.848002) (width 0.25) (layer F.Cu) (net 12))
 (segment (start 106.989445 87.083664) (end 106.989445 86.089445) (width 0.25) (layer F.Cu) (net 12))
 (segment (start 106.974998 87.848002) (end 106.974998 87.098111) (width 0.25) (layer F.Cu) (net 12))
 (segment (start 106.376369 87.885784) (end 106.376369 87.413273) (width 0.25) (layer F.Cu) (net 13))
 (segment (start 107.420585 88.93) (end 106.376369 87.885784) (width 0.25) (layer F.Cu) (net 13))
 (segment (start 106.264443 87.301347) (end 106.264443 86.735662) (width 0.25) (layer F.Cu) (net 13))
 (via (at 106.264443 86.735662) (size 0.8) (drill 0.4) (layers F.Cu B.Cu) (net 13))
 (segment (start 106.195 86.4) (end 106.195 86.666219) (width 0.25) (layer B.Cu) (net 13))
 (segment (start 106.195 86.666219) (end 106.264443 86.735662) (width 0.25) (layer B.Cu) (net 13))
 (segment (start 106.376369 87.413273) (end 106.264443 87.301347) (width 0.25) (layer F.Cu) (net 13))
 (segment (start 110.11 88.93) (end 107.420585 88.93) (width 0.25) (layer F.Cu) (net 13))
 (via (at 106.105858 90.16224) (size 0.8) (drill 0.4) (layers F.Cu B.Cu) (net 16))
 (segment (start 106.273618 90.33) (end 106.105858 90.16224) (width 0.25) (layer F.Cu) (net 16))
 (segment (start 106.195 91.44) (end 106.195 90.251382) (width 0.25) (layer B.Cu) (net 16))
 (segment (start 106.195 90.251382) (end 106.105858 90.16224) (width 0.25) (layer B.Cu) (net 16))
 (segment (start 110.11 90.33) (end 106.273618 90.33) (width 0.25) (layer F.Cu) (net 16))
 (via (at 105.3 92.5) (size 0.8) (drill 0.4) (layers F.Cu B.Cu) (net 17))
 (segment (start 104.67 93.13) (end 105.3 92.5) (width 0.25) (layer F.Cu) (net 17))
 (segment (start 100.71 93.13) (end 104.67 93.13) (width 0.25) (layer F.Cu) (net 17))
 (segment (start 106.186399 82.950011) (end 107.904987 82.950011) (width 0.25) (layer B.Cu) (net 17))
 (segment (start 105.30501 83.8314) (end 106.186399 82.950011) (width 0.25) (layer B.Cu) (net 17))
 (segment (start 107.904987 82.950011) (end 108.159999 82.694999) (width 0.25) (layer B.Cu) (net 17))
 (segment (start 105.30501 85.721986) (end 105.30501 83.8314) (width 0.25) (layer B.Cu) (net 17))
 (segment (start 105.10501 88.531778) (end 105.074998 88.501766) (width 0.25) (layer B.Cu) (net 17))
 (segment (start 105.074998 88.501766) (end 105.074998 85.951998) (width 0.25) (layer B.Cu) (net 17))
 (segment (start 105.074998 85.951998) (end 105.30501 85.721986) (width 0.25) (layer B.Cu) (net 17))
 (segment (start 105.10501 89.078014) (end 105.10501 88.531778) (width 0.25) (layer B.Cu) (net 17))
 (segment (start 105.3 92.5) (end 105.3 89.273004) (width 0.25) (layer B.Cu) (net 17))
 (segment (start 105.3 89.273004) (end 105.10501 89.078014) (width 0.25) (layer B.Cu) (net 17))
 (segment (start 100.2 93.64) (end 100.71 93.13) (width 0.25) (layer F.Cu) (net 17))
 (segment (start 100.2 97.4625) (end 100.2 93.64) (width 0.25) (layer F.Cu) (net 17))
 (via (at 101.6 102.6) (size 0.8) (drill 0.4) (layers F.Cu B.Cu) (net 17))
 (segment (start 102.05 103.05) (end 101.6 102.6) (width 0.25) (layer F.Cu) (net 17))
 (segment (start 103.425 103.05) (end 102.05 103.05) (width 0.25) (layer F.Cu) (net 17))
 (via (at 101.086006 97.556036) (size 0.8) (drill 0.4) (layers F.Cu B.Cu) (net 17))
 (segment (start 101.086006 97.548506) (end 101.086006 97.556036) (width 0.25) (layer F.Cu) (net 17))
 (segment (start 100.2 97.4625) (end 101 97.4625) (width 0.25) (layer F.Cu) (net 17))
 (segment (start 101 97.4625) (end 101.086006 97.548506) (width 0.25) (layer F.Cu) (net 17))
 (segment (start 101.086006 102.086006) (end 101.086006 98.121721) (width 0.25) (layer B.Cu) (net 17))
 (segment (start 101.6 102.6) (end 101.086006 102.086006) (width 0.25) (layer B.Cu) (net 17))
 (segment (start 101.086006 98.121721) (end 101.086006 97.556036) (width 0.25) (layer B.Cu) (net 17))
 (segment (start 103.425 103.05) (end 111.375 103.05) (width 0.25) (layer F.Cu) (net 17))
 (segment (start 114.175 85.4) (end 113.5 85.4) (width 0.25) (layer F.Cu) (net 17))
 (segment (start 114.2 85.425) (end 114.175 85.4) (width 0.25) (layer F.Cu) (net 17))
 (segment (start 114.2 89.26) (end 114.2 85.425) (width 0.25) (layer F.Cu) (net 17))
 (via (at 111.6 101.3) (size 0.8) (drill 0.4) (layers F.Cu B.Cu) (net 17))
 (segment (start 115.375001 90.689999) (end 115.375001 97.524999) (width 0.25) (layer B.Cu) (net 17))
 (segment (start 115.310001 90.624999) (end 115.375001 90.689999) (width 0.25) (layer B.Cu) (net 17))
 (segment (start 115.375001 97.524999) (end 111.6 101.3) (width 0.25) (layer B.Cu) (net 17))
 (segment (start 111.6 102.825) (end 111.375 103.05) (width 0.25) (layer F.Cu) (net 17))
 (segment (start 111.6 101.3) (end 111.6 102.825) (width 0.25) (layer F.Cu) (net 17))
 (segment (start 115.310001 90.370001) (end 114.2 89.26) (width 0.25) (layer B.Cu) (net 17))
 (segment (start 115.310001 90.624999) (end 115.310001 90.370001) (width 0.25) (layer B.Cu) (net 17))
 (segment (start 103.815002 81.774998) (end 101.76 83.83) (width 0.25) (layer F.Cu) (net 32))
 (segment (start 105.448002 81.774998) (end 103.815002 81.774998) (width 0.25) (layer F.Cu) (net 32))
 (segment (start 110.11 83.83) (end 107.503004 83.83) (width 0.25) (layer F.Cu) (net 32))
 (segment (start 101.76 83.83) (end 100.71 83.83) (width 0.25) (layer F.Cu) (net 32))
 (segment (start 107.503004 83.83) (end 105.448002 81.774998) (width 0.25) (layer F.Cu) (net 32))
 (segment (start 100.2 99.3375) (end 101 99.3375) (width 0.25) (layer F.Cu) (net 32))
 (segment (start 101.21 96.38) (end 101.21 95.33) (width 0.25) (layer F.Cu) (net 32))
 (segment (start 101 99.3375) (end 102.025001 98.312499) (width 0.25) (layer F.Cu) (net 32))
 (segment (start 102.025001 97.195001) (end 101.21 96.38) (width 0.25) (layer F.Cu) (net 32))
 (segment (start 108.89 97.1) (end 104 97.1) (width 0.25) (layer F.Cu) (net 32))
 (via (at 104 97.1) (size 0.8) (drill 0.4) (layers F.Cu B.Cu) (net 32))
 (via (at 102.025001 97.9) (size 0.8) (drill 0.4) (layers F.Cu B.Cu) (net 32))
 (segment (start 102.825001 97.1) (end 102.025001 97.9) (width 0.25) (layer B.Cu) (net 32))
 (segment (start 104 97.1) (end 102.825001 97.1) (width 0.25) (layer B.Cu) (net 32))
 (segment (start 102.025001 98.312499) (end 102.025001 97.9) (width 0.25) (layer F.Cu) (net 32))
 (segment (start 102.025001 97.9) (end 102.025001 97.195001) (width 0.25) (layer F.Cu) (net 32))
 (segment (start 110.11 83.38896) (end 110.11 83.83) (width 0.25) (layer F.Cu) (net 32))
 (segment (start 109.61 96.38) (end 109.61 95.33) (width 0.25) (layer F.Cu) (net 32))
 (segment (start 110.06 95.33) (end 109.61 95.33) (width 0.25) (layer F.Cu) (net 32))
 (segment (start 111.77 95.33) (end 110.06 95.33) (width 0.25) (layer F.Cu) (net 32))
 (segment (start 114.2 92.9) (end 111.77 95.33) (width 0.25) (layer F.Cu) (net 32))
 (segment (start 114.2 91.8) (end 114.2 92.9) (width 0.25) (layer F.Cu) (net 32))
 (segment (start 112.09896 81.4) (end 113.5 81.4) (width 0.25) (layer F.Cu) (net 32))
 (segment (start 110.11 83.38896) (end 112.09896 81.4) (width 0.25) (layer F.Cu) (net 32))
 (segment (start 115.375001 91.724999) (end 115.3 91.8) (width 0.25) (layer F.Cu) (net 32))
 (segment (start 114.10104 81.4) (end 115.375001 82.673961) (width 0.25) (layer F.Cu) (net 32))
 (segment (start 115.3 91.8) (end 114.2 91.8) (width 0.25) (layer F.Cu) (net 32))
 (segment (start 115.375001 82.673961) (end 115.375001 91.724999) (width 0.25) (layer F.Cu) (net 32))
 (segment (start 113.5 81.4) (end 114.10104 81.4) (width 0.25) (layer F.Cu) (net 32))
 (via (at 111.5 96.8) (size 0.8) (drill 0.4) (layers F.Cu B.Cu) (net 32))
 (segment (start 114.2 94.1) (end 111.5 96.8) (width 0.25) (layer B.Cu) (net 32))
 (segment (start 114.2 91.8) (end 114.2 94.1) (width 0.25) (layer B.Cu) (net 32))
 (segment (start 109.39 96.6) (end 108.89 97.1) (width 0.25) (layer F.Cu) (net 32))
 (segment (start 109.61 96.38) (end 109.39 96.6) (width 0.25) (layer F.Cu) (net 32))
 (segment (start 111.5 96.8) (end 111 97.3) (width 0.25) (layer F.Cu) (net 32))
 (segment (start 109.09 97.3) (end 108.89 97.1) (width 0.25) (layer F.Cu) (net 32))
 (segment (start 111 97.3) (end 109.09 97.3) (width 0.25) (layer F.Cu) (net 32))
 (segment (start 101.91 96.135) (end 101.91 95.33) (width 0.25) (layer F.Cu) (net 43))
 (segment (start 103.425 97.65) (end 101.91 96.135) (width 0.25) (layer F.Cu) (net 43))
 (segment (start 103.425 98.55) (end 103.425 97.65) (width 0.25) (layer F.Cu) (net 43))
 (segment (start 104.45 98.55) (end 111.375 98.55) (width 0.25) (layer F.Cu) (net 43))
 (segment (start 103.425 98.55) (end 104.45 98.55) (width 0.25) (layer F.Cu) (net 43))
 (segment (start 111.137341 85.337339) (end 111.53734 84.93734) (width 0.25) (layer F.Cu) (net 23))
 (via (at 111.53734 84.93734) (size 0.8) (drill 0.4) (layers F.Cu B.Cu) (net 23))
 (segment (start 110.11 85.43) (end 111.04468 85.43) (width 0.25) (layer F.Cu) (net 23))
 (segment (start 111.04468 85.43) (end 111.137341 85.337339) (width 0.25) (layer F.Cu) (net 23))
 (segment (start 113.5 84.4) (end 112.07468 84.4) (width 0.25) (layer B.Cu) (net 23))
 (segment (start 112.07468 84.4) (end 111.53734 84.93734) (width 0.25) (layer B.Cu) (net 23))
 (segment (start 111.849999 86.150001) (end 111.8 86.2) (width 0.25) (layer B.Cu) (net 24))
 (segment (start 114.185001 86.150001) (end 111.849999 86.150001) (width 0.25) (layer B.Cu) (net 24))
 (segment (start 114.250001 86.085001) (end 114.185001 86.150001) (width 0.25) (layer B.Cu) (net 24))
 (segment (start 114.250001 84.039999) (end 114.250001 86.085001) (width 0.25) (layer B.Cu) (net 24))
 (segment (start 113.139999 83.649999) (end 113.860001 83.649999) (width 0.25) (layer B.Cu) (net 24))
 (segment (start 113.389998 83.4) (end 113.139999 83.649999) (width 0.25) (layer B.Cu) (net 24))
 (segment (start 113.5 83.4) (end 113.389998 83.4) (width 0.25) (layer B.Cu) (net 24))
 (via (at 111.8 86.2) (size 0.8) (drill 0.4) (layers F.Cu B.Cu) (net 24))
 (segment (start 113.860001 83.649999) (end 114.250001 84.039999) (width 0.25) (layer B.Cu) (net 24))
 (segment (start 110.18 86.2) (end 110.11 86.13) (width 0.25) (layer F.Cu) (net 24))
 (segment (start 111.8 86.2) (end 110.18 86.2) (width 0.25) (layer F.Cu) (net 24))
 (segment (start 113.5 82.4) (end 112.89896 82.4) (width 0.25) (layer F.Cu) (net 25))
 (segment (start 111.455001 87.125001) (end 111.16 86.83) (width 0.25) (layer F.Cu) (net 25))
 (segment (start 111.948001 87.125001) (end 111.455001 87.125001) (width 0.25) (layer F.Cu) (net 25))
 (segment (start 112.525001 86.548001) (end 111.948001 87.125001) (width 0.25) (layer F.Cu) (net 25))
 (segment (start 111.16 86.83) (end 110.11 86.83) (width 0.25) (layer F.Cu) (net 25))
 (segment (start 112.525001 82.773959) (end 112.525001 86.548001) (width 0.25) (layer F.Cu) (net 25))
 (segment (start 112.89896 82.4) (end 112.525001 82.773959) (width 0.25) (layer F.Cu) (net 25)))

